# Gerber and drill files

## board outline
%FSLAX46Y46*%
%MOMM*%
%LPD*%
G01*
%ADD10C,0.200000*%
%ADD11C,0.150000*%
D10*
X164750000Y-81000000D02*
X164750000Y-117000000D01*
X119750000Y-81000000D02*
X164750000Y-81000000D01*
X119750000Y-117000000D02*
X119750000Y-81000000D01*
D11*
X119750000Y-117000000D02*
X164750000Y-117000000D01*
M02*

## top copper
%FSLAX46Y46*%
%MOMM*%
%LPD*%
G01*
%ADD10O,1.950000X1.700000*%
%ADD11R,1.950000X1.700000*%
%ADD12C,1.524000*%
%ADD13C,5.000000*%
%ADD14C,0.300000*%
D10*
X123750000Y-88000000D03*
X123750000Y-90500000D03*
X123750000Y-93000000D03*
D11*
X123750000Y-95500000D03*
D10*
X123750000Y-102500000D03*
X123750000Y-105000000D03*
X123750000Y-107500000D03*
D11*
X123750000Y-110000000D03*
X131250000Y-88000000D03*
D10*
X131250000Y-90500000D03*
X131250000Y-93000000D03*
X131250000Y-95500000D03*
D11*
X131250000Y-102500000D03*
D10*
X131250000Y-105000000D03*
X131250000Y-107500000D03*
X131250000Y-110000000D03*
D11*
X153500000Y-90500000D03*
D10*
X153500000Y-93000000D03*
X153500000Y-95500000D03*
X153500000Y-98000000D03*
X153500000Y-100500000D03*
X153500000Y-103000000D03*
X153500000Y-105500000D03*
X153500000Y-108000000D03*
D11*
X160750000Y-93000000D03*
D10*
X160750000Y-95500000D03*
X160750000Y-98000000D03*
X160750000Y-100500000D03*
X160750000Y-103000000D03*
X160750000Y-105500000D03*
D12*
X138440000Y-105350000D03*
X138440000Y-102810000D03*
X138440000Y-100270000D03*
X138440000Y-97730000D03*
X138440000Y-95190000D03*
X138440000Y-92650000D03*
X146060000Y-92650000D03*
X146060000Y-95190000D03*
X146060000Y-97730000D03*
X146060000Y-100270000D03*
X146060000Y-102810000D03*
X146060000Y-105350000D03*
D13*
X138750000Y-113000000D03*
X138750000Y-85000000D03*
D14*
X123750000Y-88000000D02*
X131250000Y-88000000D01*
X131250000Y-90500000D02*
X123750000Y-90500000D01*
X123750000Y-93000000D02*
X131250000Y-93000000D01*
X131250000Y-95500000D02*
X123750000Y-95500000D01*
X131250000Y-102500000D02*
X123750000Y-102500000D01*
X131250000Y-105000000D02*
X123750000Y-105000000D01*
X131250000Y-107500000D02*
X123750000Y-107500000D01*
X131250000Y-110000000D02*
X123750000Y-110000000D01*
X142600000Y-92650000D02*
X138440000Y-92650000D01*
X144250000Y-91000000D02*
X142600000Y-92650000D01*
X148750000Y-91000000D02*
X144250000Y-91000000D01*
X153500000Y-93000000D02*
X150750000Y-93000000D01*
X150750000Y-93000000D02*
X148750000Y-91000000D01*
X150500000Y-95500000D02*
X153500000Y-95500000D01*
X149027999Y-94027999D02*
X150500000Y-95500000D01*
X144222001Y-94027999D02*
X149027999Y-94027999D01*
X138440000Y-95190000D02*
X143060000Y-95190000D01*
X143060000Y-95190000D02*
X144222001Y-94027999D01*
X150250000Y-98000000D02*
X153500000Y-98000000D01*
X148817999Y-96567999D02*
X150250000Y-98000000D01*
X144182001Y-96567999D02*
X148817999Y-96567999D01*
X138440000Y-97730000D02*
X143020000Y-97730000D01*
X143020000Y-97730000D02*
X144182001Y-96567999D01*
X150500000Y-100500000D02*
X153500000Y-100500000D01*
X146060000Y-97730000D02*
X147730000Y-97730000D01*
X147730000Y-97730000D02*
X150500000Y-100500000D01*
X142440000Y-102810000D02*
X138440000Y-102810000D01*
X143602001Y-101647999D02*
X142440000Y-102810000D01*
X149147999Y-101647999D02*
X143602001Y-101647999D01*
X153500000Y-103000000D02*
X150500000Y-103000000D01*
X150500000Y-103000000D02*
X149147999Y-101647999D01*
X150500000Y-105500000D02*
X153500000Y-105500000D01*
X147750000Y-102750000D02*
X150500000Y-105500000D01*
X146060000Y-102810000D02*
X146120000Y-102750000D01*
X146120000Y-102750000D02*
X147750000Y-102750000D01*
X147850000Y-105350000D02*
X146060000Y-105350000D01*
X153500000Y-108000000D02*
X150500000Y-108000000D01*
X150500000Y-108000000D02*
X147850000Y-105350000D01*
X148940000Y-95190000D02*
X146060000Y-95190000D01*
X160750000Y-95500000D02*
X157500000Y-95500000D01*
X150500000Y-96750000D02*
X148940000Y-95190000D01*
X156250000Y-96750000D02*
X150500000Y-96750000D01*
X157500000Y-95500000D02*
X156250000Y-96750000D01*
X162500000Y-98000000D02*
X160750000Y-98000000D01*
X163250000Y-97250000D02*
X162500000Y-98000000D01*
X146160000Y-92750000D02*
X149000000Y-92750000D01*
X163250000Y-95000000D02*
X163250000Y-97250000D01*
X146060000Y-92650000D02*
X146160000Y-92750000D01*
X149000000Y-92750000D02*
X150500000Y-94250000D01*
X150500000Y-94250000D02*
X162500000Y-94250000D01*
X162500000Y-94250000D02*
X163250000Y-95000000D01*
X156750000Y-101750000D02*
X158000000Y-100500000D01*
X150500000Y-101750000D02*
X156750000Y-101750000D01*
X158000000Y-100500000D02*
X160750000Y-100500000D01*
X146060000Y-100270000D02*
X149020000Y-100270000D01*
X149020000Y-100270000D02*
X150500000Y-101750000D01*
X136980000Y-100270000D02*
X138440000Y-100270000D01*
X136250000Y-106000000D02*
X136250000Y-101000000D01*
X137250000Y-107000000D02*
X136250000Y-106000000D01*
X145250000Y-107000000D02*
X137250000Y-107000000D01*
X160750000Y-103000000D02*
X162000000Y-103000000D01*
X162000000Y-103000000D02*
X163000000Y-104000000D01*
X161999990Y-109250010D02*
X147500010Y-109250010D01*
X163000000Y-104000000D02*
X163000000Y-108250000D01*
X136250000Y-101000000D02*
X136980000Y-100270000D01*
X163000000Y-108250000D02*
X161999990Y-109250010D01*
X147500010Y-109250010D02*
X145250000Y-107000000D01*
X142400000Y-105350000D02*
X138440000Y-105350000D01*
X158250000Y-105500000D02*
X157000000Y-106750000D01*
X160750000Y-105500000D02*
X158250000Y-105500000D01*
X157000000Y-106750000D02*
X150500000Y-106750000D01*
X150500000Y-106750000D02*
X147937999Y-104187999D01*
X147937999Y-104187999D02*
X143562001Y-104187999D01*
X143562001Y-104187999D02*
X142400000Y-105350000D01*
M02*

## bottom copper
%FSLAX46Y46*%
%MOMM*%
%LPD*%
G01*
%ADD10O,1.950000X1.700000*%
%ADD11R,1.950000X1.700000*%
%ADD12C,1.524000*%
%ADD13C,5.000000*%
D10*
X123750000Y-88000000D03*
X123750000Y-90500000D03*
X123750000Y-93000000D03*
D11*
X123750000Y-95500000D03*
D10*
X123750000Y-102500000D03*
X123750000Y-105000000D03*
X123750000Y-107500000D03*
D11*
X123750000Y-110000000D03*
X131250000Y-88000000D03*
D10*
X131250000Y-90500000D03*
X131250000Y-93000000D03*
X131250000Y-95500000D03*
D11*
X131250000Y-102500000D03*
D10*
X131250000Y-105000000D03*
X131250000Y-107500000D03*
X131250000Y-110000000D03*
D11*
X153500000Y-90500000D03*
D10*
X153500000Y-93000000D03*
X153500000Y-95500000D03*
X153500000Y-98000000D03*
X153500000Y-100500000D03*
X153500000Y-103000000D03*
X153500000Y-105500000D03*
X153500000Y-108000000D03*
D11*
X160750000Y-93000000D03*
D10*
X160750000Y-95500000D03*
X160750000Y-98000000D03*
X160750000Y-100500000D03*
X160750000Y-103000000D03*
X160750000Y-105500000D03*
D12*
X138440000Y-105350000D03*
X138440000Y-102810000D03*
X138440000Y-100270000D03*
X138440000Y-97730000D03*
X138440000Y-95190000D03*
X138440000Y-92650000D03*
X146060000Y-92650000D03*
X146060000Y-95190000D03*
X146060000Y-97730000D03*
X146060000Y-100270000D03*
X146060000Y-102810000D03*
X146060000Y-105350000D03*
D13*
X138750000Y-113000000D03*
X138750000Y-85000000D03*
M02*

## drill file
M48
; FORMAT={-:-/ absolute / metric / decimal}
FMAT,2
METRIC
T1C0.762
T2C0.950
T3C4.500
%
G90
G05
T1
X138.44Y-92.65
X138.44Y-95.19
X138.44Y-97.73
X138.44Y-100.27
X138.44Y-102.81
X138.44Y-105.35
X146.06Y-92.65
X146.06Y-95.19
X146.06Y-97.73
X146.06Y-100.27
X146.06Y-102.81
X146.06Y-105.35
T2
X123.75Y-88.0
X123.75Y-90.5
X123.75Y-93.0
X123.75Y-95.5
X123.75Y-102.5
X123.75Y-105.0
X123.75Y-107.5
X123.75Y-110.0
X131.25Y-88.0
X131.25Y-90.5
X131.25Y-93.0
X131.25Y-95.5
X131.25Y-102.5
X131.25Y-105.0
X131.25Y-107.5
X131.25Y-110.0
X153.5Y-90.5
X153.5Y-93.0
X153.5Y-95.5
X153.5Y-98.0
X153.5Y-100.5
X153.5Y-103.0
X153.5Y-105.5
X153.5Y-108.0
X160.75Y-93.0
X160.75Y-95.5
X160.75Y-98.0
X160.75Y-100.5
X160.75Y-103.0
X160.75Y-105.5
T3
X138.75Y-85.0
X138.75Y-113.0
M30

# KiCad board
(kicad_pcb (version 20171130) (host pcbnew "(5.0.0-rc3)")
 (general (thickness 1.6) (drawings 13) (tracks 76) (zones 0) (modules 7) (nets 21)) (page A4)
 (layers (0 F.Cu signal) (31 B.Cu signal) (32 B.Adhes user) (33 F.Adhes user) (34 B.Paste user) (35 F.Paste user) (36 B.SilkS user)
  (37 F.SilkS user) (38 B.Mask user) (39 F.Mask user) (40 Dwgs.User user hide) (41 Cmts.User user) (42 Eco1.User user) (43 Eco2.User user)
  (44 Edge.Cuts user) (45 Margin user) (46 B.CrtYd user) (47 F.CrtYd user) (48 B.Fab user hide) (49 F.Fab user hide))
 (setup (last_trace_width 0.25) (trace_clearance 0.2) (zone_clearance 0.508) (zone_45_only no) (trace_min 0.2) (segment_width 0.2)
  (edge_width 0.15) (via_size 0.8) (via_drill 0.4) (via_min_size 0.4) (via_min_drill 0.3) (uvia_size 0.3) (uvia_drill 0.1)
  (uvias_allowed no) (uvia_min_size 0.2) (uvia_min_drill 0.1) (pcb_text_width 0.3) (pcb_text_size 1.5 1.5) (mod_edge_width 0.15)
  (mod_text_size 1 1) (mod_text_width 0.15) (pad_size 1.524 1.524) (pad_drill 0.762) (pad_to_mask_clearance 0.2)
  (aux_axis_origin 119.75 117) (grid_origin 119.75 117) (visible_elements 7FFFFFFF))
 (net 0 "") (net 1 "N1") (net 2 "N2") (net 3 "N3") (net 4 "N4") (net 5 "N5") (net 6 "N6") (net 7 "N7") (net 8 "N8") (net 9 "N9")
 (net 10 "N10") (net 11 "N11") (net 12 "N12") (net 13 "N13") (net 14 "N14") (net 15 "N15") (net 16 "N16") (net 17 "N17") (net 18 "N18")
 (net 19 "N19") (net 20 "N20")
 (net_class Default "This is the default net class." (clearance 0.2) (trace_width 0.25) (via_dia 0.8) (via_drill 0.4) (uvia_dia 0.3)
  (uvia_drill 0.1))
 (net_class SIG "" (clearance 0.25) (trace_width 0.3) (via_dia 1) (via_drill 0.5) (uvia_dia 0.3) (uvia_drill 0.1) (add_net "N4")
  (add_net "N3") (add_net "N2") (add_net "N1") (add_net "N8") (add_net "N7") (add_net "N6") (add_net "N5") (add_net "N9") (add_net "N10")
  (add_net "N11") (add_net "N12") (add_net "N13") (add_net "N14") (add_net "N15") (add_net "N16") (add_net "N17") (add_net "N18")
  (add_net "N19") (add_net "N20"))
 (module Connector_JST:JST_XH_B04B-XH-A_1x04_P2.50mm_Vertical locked (layer B.Cu) (at 123.75 95.5 90)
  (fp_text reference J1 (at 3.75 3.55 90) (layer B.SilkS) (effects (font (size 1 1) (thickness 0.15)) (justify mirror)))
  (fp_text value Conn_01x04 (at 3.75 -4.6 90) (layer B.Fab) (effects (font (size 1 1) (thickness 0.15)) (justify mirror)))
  (pad 4 thru_hole oval (at 7.5 0 90) (size 1.7 1.95) (drill 0.95) (layers *.Cu *.Mask) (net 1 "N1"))
  (pad 3 thru_hole oval (at 5 0 90) (size 1.7 1.95) (drill 0.95) (layers *.Cu *.Mask) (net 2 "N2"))
  (pad 2 thru_hole oval (at 2.5 0 90) (size 1.7 1.95) (drill 0.95) (layers *.Cu *.Mask) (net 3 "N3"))
  (pad 1 thru_hole rect (at 0 0 90) (size 1.7 1.95) (drill 0.95) (layers *.Cu *.Mask) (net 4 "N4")))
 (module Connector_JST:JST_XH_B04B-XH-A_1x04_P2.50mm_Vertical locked (layer B.Cu) (at 123.75 110 90)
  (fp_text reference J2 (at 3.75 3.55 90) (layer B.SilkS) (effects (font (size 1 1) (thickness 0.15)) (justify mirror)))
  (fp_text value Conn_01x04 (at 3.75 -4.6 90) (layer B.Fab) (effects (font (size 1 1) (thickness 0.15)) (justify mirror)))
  (pad 4 thru_hole oval (at 7.5 0 90) (size 1.7 1.95) (drill 0.95) (layers *.Cu *.Mask) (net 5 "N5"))
  (pad 3 thru_hole oval (at 5 0 90) (size 1.7 1.95) (drill 0.95) (layers *.Cu *.Mask) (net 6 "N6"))
  (pad 2 thru_hole oval (at 2.5 0 90) (size 1.7 1.95) (drill 0.95) (layers *.Cu *.Mask) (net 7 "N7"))
  (pad 1 thru_hole rect (at 0 0 90) (size 1.7 1.95) (drill 0.95) (layers *.Cu *.Mask) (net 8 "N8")))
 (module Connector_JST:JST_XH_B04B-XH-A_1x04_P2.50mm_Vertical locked (layer F.Cu) (at 131.25 88 270)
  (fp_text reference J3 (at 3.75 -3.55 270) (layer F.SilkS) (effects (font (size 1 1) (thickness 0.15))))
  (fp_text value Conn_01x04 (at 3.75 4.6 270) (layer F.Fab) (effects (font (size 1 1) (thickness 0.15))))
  (pad 1 thru_hole rect (at 0 0 270) (size 1.7 1.95) (drill 0.95) (layers *.Cu *.Mask) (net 1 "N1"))
  (pad 2 thru_hole oval (at 2.5 0 270) (size 1.7 1.95) (drill 0.95) (layers *.Cu *.Mask) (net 2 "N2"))
  (pad 3 thru_hole oval (at 5 0 270) (size 1.7 1.95) (drill 0.95) (layers *.Cu *.Mask) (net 3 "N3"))
  (pad 4 thru_hole oval (at 7.5 0 270) (size 1.7 1.95) (drill 0.95) (layers *.Cu *.Mask) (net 4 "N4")))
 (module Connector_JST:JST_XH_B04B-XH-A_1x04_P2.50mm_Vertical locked (layer F.Cu) (at 131.25 102.5 270)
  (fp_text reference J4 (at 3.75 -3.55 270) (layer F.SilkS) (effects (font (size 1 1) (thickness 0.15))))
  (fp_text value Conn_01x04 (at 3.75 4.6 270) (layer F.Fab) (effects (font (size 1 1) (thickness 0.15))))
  (pad 1 thru_hole rect (at 0 0 270) (size 1.7 1.95) (drill 0.95) (layers *.Cu *.Mask) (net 5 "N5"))
  (pad 2 thru_hole oval (at 2.5 0 270) (size 1.7 1.95) (drill 0.95) (layers *.Cu *.Mask) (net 6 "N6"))
  (pad 3 thru_hole oval (at 5 0 270) (size 1.7 1.95) (drill 0.95) (layers *.Cu *.Mask) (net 7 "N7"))
  (pad 4 thru_hole oval (at 7.5 0 270) (size 1.7 1.95) (drill 0.95) (layers *.Cu *.Mask) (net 8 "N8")))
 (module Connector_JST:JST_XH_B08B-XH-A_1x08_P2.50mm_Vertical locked (layer F.Cu) (at 153.5 90.5 270)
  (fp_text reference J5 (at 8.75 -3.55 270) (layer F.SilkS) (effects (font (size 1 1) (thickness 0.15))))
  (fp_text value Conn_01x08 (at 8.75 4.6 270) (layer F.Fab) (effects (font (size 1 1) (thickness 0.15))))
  (pad 1 thru_hole rect (at 0 0 270) (size 1.7 1.95) (drill 0.95) (layers *.Cu *.Mask))
  (pad 2 thru_hole oval (at 2.5 0 270) (size 1.7 1.95) (drill 0.95) (layers *.Cu *.Mask) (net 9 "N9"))
  (pad 3 thru_hole oval (at 5 0 270) (size 1.7 1.95) (drill 0.95) (layers *.Cu *.Mask) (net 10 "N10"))
  (pad 4 thru_hole oval (at 7.5 0 270) (size 1.7 1.95) (drill 0.95) (layers *.Cu *.Mask) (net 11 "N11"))
  (pad 5 thru_hole oval (at 10 0 270) (size 1.7 1.95) (drill 0.95) (layers *.Cu *.Mask) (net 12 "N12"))
  (pad 6 thru_hole oval (at 12.5 0 270) (size 1.7 1.95) (drill 0.95) (layers *.Cu *.Mask) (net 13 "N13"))
  (pad 7 thru_hole oval (at 15 0 270) (size 1.7 1.95) (drill 0.95) (layers *.Cu *.Mask) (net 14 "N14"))
  (pad 8 thru_hole oval (at 17.5 0 270) (size 1.7 1.95) (drill 0.95) (layers *.Cu *.Mask) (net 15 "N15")))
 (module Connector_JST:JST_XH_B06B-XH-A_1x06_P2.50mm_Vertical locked (layer F.Cu) (at 160.75 93 270)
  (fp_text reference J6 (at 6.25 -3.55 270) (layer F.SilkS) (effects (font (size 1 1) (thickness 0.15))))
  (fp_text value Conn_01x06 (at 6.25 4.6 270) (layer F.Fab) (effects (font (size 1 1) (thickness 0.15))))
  (pad 1 thru_hole rect (at 0 0 270) (size 1.7 1.95) (drill 0.95) (layers *.Cu *.Mask))
  (pad 2 thru_hole oval (at 2.5 0 270) (size 1.7 1.95) (drill 0.95) (layers *.Cu *.Mask) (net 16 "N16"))
  (pad 3 thru_hole oval (at 5 0 270) (size 1.7 1.95) (drill 0.95) (layers *.Cu *.Mask) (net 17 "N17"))
  (pad 4 thru_hole oval (at 7.5 0 270) (size 1.7 1.95) (drill 0.95) (layers *.Cu *.Mask) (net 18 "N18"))
  (pad 5 thru_hole oval (at 10 0 270) (size 1.7 1.95) (drill 0.95) (layers *.Cu *.Mask) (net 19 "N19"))
  (pad 6 thru_hole oval (at 12.5 0 270) (size 1.7 1.95) (drill 0.95) (layers *.Cu *.Mask) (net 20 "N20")))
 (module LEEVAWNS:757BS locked (layer B.Cu) (at 142.25 99)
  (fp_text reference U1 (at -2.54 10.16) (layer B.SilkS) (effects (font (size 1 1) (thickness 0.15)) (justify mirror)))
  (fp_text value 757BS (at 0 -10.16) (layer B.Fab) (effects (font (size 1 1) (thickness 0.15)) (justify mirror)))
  (pad 1 thru_hole circle (at -3.81 6.35) (size 1.524 1.524) (drill 0.762) (layers *.Cu *.Mask) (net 20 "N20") (thermal_width 0.5)
   (thermal_gap 0.5))
  (pad 2 thru_hole circle (at -3.81 3.81) (size 1.524 1.524) (drill 0.762) (layers *.Cu *.Mask) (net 13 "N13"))
  (pad 3 thru_hole circle (at -3.81 1.27) (size 1.524 1.524) (drill 0.762) (layers *.Cu *.Mask) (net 19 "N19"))
  (pad 4 thru_hole circle (at -3.81 -1.27) (size 1.524 1.524) (drill 0.762) (layers *.Cu *.Mask) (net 11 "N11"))
  (pad 5 thru_hole circle (at -3.81 -3.81) (size 1.524 1.524) (drill 0.762) (layers *.Cu *.Mask) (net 10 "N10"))
  (pad 6 thru_hole circle (at -3.81 -6.35) (size 1.524 1.524) (drill 0.762) (layers *.Cu *.Mask) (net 9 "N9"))
  (pad 7 thru_hole circle (at 3.81 -6.35) (size 1.524 1.524) (drill 0.762) (layers *.Cu *.Mask) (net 17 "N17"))
  (pad 8 thru_hole circle (at 3.81 -3.81) (size 1.524 1.524) (drill 0.762) (layers *.Cu *.Mask) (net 16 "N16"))
  (pad 9 thru_hole circle (at 3.81 -1.27) (size 1.524 1.524) (drill 0.762) (layers *.Cu *.Mask) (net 12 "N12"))
  (pad 10 thru_hole circle (at 3.81 1.27) (size 1.524 1.524) (drill 0.762) (layers *.Cu *.Mask) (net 18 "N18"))
  (pad 11 thru_hole circle (at 3.81 3.81) (size 1.524 1.524) (drill 0.762) (layers *.Cu *.Mask) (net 14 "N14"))
  (pad 12 thru_hole circle (at 3.81 6.35) (size 1.524 1.524) (drill 0.762) (layers *.Cu *.Mask) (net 15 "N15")))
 (gr_line (start 164.75 81) (end 164.75 117) (layer Edge.Cuts) (width 0.2))
 (gr_line (start 119.75 81) (end 164.75 81) (layer Edge.Cuts) (width 0.2))
 (gr_line (start 119.75 117) (end 119.75 81) (layer Edge.Cuts) (width 0.2))
 (gr_line (start 119.75 117) (end 164.75 117) (layer Edge.Cuts) (width 0.15))
 (via (at 138.75 113) (size 5) (drill 4.5) (layers F.Cu B.Cu) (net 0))
 (via (at 138.75 85) (size 5) (drill 4.5) (layers F.Cu B.Cu) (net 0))
 (segment (start 123.75 88) (end 131.25 88) (width 0.3) (layer F.Cu) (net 1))
 (segment (start 131.25 90.5) (end 123.75 90.5) (width 0.3) (layer F.Cu) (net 2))
 (segment (start 123.75 93) (end 131.25 93) (width 0.3) (layer F.Cu) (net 3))
 (segment (start 131.25 95.5) (end 123.75 95.5) (width 0.3) (layer F.Cu) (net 4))
 (segment (start 131.25 102.5) (end 123.75 102.5) (width 0.3) (layer F.Cu) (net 5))
 (segment (start 131.25 105) (end 123.75 105) (width 0.3) (layer F.Cu) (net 6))
 (segment (start 131.25 107.5) (end 123.75 107.5) (width 0.3) (layer F.Cu) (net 7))
 (segment (start 131.25 110) (end 123.75 110) (width 0.3) (layer F.Cu) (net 8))
 (segment (start 142.6 92.65) (end 138.44 92.65) (width 0.3) (layer F.Cu) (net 9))
 (segment (start 144.25 91) (end 142.6 92.65) (width 0.3) (layer F.Cu) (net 9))
 (segment (start 148.75 91) (end 144.25 91) (width 0.3) (layer F.Cu) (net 9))
 (segment (start 153.5 93) (end 150.75 93) (width 0.3) (layer F.Cu) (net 9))
 (segment (start 150.75 93) (end 148.75 91) (width 0.3) (layer F.Cu) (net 9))
 (segment (start 150.5 95.5) (end 153.5 95.5) (width 0.3) (layer F.Cu) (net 10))
 (segment (start 149.027999 94.027999) (end 150.5 95.5) (width 0.3) (layer F.Cu) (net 10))
 (segment (start 144.222001 94.027999) (end 149.027999 94.027999) (width 0.3) (layer F.Cu) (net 10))
 (segment (start 138.44 95.19) (end 143.06 95.19) (width 0.3) (layer F.Cu) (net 10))
 (segment (start 143.06 95.19) (end 144.222001 94.027999) (width 0.3) (layer F.Cu) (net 10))
 (segment (start 150.25 98) (end 153.5 98) (width 0.3) (layer F.Cu) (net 11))
 (segment (start 148.817999 96.567999) (end 150.25 98) (width 0.3) (layer F.Cu) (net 11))
 (segment (start 144.182001 96.567999) (end 148.817999 96.567999) (width 0.3) (layer F.Cu) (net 11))
 (segment (start 138.44 97.73) (end 143.02 97.73) (width 0.3) (layer F.Cu) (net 11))
 (segment (start 143.02 97.73) (end 144.182001 96.567999) (width 0.3) (layer F.Cu) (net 11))
 (segment (start 150.5 100.5) (end 153.5 100.5) (width 0.3) (layer F.Cu) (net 12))
 (segment (start 146.06 97.73) (end 147.73 97.73) (width 0.3) (layer F.Cu) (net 12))
 (segment (start 147.73 97.73) (end 150.5 100.5) (width 0.3) (layer F.Cu) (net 12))
 (segment (start 142.44 102.81) (end 138.44 102.81) (width 0.3) (layer F.Cu) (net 13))
 (segment (start 143.602001 101.647999) (end 142.44 102.81) (width 0.3) (layer F.Cu) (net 13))
 (segment (start 149.147999 101.647999) (end 143.602001 101.647999) (width 0.3) (layer F.Cu) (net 13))
 (segment (start 153.5 103) (end 150.5 103) (width 0.3) (layer F.Cu) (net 13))
 (segment (start 150.5 103) (end 149.147999 101.647999) (width 0.3) (layer F.Cu) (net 13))
 (segment (start 150.5 105.5) (end 153.5 105.5) (width 0.3) (layer F.Cu) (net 14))
 (segment (start 147.75 102.75) (end 150.5 105.5) (width 0.3) (layer F.Cu) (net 14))
 (segment (start 146.06 102.81) (end 146.12 102.75) (width 0.3) (layer F.Cu) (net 14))
 (segment (start 146.12 102.75) (end 147.75 102.75) (width 0.3) (layer F.Cu) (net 14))
 (segment (start 147.85 105.35) (end 146.06 105.35) (width 0.3) (layer F.Cu) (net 15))
 (segment (start 153.5 108) (end 150.5 108) (width 0.3) (layer F.Cu) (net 15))
 (segment (start 150.5 108) (end 147.85 105.35) (width 0.3) (layer F.Cu) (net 15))
 (segment (start 148.94 95.19) (end 146.06 95.19) (width 0.3) (layer F.Cu) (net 16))
 (segment (start 160.75 95.5) (end 157.5 95.5) (width 0.3) (layer F.Cu) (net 16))
 (segment (start 150.5 96.75) (end 148.94 95.19) (width 0.3) (layer F.Cu) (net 16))
 (segment (start 156.25 96.75) (end 150.5 96.75) (width 0.3) (layer F.Cu) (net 16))
 (segment (start 157.5 95.5) (end 156.25 96.75) (width 0.3) (layer F.Cu) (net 16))
 (segment (start 162.5 98) (end 160.75 98) (width 0.3) (layer F.Cu) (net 17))
 (segment (start 163.25 97.25) (end 162.5 98) (width 0.3) (layer F.Cu) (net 17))
 (segment (start 146.16 92.75) (end 149 92.75) (width 0.3) (layer F.Cu) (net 17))
 (segment (start 163.25 95) (end 163.25 97.25) (width 0.3) (layer F.Cu) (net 17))
 (segment (start 146.06 92.65) (end 146.16 92.75) (width 0.3) (layer F.Cu) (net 17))
 (segment (start 149 92.75) (end 150.5 94.25) (width 0.3) (layer F.Cu) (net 17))
 (segment (start 150.5 94.25) (end 162.5 94.25) (width 0.3) (layer F.Cu) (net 17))
 (segment (start 162.5 94.25) (end 163.25 95) (width 0.3) (layer F.Cu) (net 17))
 (segment (start 156.75 101.75) (end 158 100.5) (width 0.3) (layer F.Cu) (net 18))
 (segment (start 150.5 101.75) (end 156.75 101.75) (width 0.3) (layer F.Cu) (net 18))
 (segment (start 158 100.5) (end 160.75 100.5) (width 0.3) (layer F.Cu) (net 18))
 (segment (start 146.06 100.27) (end 149.02 100.27) (width 0.3) (layer F.Cu) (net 18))
 (segment (start 149.02 100.27) (end 150.5 101.75) (width 0.3) (layer F.Cu) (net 18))
 (segment (start 136.98 100.27) (end 138.44 100.27) (width 0.3) (layer F.Cu) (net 19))
 (segment (start 136.25 106) (end 136.25 101) (width 0.3) (layer F.Cu) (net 19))
 (segment (start 137.25 107) (end 136.25 106) (width 0.3) (layer F.Cu) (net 19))
 (segment (start 145.25 107) (end 137.25 107) (width 0.3) (layer F.Cu) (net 19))
 (segment (start 160.75 103) (end 162 103) (width 0.3) (layer F.Cu) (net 19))
 (segment (start 162 103) (end 163 104) (width 0.3) (layer F.Cu) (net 19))
 (segment (start 161.99999 109.25001) (end 147.50001 109.25001) (width 0.3) (layer F.Cu) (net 19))
 (segment (start 163 104) (end 163 108.25) (width 0.3) (layer F.Cu) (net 19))
 (segment (start 136.25 101) (end 136.98 100.27) (width 0.3) (layer F.Cu) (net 19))
 (segment (start 163 108.25) (end 161.99999 109.25001) (width 0.3) (layer F.Cu) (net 19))
 (segment (start 147.50001 109.25001) (end 145.25 107) (width 0.3) (layer F.Cu) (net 19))
 (segment (start 142.4 105.35) (end 138.44 105.35) (width 0.3) (layer F.Cu) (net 20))
 (segment (start 158.25 105.5) (end 157 106.75) (width 0.3) (layer F.Cu) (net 20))
 (segment (start 160.75 105.5) (end 158.25 105.5) (width 0.3) (layer F.Cu) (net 20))
 (segment (start 157 106.75) (end 150.5 106.75) (width 0.3) (layer F.Cu) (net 20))
 (segment (start 150.5 106.75) (end 147.937999 104.187999) (width 0.3) (layer F.Cu) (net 20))
 (segment (start 147.937999 104.187999) (end 143.562001 104.187999) (width 0.3) (layer F.Cu) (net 20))
 (segment (start 143.562001 104.187999) (end 142.4 105.35) (width 0.3) (layer F.Cu) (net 20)))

